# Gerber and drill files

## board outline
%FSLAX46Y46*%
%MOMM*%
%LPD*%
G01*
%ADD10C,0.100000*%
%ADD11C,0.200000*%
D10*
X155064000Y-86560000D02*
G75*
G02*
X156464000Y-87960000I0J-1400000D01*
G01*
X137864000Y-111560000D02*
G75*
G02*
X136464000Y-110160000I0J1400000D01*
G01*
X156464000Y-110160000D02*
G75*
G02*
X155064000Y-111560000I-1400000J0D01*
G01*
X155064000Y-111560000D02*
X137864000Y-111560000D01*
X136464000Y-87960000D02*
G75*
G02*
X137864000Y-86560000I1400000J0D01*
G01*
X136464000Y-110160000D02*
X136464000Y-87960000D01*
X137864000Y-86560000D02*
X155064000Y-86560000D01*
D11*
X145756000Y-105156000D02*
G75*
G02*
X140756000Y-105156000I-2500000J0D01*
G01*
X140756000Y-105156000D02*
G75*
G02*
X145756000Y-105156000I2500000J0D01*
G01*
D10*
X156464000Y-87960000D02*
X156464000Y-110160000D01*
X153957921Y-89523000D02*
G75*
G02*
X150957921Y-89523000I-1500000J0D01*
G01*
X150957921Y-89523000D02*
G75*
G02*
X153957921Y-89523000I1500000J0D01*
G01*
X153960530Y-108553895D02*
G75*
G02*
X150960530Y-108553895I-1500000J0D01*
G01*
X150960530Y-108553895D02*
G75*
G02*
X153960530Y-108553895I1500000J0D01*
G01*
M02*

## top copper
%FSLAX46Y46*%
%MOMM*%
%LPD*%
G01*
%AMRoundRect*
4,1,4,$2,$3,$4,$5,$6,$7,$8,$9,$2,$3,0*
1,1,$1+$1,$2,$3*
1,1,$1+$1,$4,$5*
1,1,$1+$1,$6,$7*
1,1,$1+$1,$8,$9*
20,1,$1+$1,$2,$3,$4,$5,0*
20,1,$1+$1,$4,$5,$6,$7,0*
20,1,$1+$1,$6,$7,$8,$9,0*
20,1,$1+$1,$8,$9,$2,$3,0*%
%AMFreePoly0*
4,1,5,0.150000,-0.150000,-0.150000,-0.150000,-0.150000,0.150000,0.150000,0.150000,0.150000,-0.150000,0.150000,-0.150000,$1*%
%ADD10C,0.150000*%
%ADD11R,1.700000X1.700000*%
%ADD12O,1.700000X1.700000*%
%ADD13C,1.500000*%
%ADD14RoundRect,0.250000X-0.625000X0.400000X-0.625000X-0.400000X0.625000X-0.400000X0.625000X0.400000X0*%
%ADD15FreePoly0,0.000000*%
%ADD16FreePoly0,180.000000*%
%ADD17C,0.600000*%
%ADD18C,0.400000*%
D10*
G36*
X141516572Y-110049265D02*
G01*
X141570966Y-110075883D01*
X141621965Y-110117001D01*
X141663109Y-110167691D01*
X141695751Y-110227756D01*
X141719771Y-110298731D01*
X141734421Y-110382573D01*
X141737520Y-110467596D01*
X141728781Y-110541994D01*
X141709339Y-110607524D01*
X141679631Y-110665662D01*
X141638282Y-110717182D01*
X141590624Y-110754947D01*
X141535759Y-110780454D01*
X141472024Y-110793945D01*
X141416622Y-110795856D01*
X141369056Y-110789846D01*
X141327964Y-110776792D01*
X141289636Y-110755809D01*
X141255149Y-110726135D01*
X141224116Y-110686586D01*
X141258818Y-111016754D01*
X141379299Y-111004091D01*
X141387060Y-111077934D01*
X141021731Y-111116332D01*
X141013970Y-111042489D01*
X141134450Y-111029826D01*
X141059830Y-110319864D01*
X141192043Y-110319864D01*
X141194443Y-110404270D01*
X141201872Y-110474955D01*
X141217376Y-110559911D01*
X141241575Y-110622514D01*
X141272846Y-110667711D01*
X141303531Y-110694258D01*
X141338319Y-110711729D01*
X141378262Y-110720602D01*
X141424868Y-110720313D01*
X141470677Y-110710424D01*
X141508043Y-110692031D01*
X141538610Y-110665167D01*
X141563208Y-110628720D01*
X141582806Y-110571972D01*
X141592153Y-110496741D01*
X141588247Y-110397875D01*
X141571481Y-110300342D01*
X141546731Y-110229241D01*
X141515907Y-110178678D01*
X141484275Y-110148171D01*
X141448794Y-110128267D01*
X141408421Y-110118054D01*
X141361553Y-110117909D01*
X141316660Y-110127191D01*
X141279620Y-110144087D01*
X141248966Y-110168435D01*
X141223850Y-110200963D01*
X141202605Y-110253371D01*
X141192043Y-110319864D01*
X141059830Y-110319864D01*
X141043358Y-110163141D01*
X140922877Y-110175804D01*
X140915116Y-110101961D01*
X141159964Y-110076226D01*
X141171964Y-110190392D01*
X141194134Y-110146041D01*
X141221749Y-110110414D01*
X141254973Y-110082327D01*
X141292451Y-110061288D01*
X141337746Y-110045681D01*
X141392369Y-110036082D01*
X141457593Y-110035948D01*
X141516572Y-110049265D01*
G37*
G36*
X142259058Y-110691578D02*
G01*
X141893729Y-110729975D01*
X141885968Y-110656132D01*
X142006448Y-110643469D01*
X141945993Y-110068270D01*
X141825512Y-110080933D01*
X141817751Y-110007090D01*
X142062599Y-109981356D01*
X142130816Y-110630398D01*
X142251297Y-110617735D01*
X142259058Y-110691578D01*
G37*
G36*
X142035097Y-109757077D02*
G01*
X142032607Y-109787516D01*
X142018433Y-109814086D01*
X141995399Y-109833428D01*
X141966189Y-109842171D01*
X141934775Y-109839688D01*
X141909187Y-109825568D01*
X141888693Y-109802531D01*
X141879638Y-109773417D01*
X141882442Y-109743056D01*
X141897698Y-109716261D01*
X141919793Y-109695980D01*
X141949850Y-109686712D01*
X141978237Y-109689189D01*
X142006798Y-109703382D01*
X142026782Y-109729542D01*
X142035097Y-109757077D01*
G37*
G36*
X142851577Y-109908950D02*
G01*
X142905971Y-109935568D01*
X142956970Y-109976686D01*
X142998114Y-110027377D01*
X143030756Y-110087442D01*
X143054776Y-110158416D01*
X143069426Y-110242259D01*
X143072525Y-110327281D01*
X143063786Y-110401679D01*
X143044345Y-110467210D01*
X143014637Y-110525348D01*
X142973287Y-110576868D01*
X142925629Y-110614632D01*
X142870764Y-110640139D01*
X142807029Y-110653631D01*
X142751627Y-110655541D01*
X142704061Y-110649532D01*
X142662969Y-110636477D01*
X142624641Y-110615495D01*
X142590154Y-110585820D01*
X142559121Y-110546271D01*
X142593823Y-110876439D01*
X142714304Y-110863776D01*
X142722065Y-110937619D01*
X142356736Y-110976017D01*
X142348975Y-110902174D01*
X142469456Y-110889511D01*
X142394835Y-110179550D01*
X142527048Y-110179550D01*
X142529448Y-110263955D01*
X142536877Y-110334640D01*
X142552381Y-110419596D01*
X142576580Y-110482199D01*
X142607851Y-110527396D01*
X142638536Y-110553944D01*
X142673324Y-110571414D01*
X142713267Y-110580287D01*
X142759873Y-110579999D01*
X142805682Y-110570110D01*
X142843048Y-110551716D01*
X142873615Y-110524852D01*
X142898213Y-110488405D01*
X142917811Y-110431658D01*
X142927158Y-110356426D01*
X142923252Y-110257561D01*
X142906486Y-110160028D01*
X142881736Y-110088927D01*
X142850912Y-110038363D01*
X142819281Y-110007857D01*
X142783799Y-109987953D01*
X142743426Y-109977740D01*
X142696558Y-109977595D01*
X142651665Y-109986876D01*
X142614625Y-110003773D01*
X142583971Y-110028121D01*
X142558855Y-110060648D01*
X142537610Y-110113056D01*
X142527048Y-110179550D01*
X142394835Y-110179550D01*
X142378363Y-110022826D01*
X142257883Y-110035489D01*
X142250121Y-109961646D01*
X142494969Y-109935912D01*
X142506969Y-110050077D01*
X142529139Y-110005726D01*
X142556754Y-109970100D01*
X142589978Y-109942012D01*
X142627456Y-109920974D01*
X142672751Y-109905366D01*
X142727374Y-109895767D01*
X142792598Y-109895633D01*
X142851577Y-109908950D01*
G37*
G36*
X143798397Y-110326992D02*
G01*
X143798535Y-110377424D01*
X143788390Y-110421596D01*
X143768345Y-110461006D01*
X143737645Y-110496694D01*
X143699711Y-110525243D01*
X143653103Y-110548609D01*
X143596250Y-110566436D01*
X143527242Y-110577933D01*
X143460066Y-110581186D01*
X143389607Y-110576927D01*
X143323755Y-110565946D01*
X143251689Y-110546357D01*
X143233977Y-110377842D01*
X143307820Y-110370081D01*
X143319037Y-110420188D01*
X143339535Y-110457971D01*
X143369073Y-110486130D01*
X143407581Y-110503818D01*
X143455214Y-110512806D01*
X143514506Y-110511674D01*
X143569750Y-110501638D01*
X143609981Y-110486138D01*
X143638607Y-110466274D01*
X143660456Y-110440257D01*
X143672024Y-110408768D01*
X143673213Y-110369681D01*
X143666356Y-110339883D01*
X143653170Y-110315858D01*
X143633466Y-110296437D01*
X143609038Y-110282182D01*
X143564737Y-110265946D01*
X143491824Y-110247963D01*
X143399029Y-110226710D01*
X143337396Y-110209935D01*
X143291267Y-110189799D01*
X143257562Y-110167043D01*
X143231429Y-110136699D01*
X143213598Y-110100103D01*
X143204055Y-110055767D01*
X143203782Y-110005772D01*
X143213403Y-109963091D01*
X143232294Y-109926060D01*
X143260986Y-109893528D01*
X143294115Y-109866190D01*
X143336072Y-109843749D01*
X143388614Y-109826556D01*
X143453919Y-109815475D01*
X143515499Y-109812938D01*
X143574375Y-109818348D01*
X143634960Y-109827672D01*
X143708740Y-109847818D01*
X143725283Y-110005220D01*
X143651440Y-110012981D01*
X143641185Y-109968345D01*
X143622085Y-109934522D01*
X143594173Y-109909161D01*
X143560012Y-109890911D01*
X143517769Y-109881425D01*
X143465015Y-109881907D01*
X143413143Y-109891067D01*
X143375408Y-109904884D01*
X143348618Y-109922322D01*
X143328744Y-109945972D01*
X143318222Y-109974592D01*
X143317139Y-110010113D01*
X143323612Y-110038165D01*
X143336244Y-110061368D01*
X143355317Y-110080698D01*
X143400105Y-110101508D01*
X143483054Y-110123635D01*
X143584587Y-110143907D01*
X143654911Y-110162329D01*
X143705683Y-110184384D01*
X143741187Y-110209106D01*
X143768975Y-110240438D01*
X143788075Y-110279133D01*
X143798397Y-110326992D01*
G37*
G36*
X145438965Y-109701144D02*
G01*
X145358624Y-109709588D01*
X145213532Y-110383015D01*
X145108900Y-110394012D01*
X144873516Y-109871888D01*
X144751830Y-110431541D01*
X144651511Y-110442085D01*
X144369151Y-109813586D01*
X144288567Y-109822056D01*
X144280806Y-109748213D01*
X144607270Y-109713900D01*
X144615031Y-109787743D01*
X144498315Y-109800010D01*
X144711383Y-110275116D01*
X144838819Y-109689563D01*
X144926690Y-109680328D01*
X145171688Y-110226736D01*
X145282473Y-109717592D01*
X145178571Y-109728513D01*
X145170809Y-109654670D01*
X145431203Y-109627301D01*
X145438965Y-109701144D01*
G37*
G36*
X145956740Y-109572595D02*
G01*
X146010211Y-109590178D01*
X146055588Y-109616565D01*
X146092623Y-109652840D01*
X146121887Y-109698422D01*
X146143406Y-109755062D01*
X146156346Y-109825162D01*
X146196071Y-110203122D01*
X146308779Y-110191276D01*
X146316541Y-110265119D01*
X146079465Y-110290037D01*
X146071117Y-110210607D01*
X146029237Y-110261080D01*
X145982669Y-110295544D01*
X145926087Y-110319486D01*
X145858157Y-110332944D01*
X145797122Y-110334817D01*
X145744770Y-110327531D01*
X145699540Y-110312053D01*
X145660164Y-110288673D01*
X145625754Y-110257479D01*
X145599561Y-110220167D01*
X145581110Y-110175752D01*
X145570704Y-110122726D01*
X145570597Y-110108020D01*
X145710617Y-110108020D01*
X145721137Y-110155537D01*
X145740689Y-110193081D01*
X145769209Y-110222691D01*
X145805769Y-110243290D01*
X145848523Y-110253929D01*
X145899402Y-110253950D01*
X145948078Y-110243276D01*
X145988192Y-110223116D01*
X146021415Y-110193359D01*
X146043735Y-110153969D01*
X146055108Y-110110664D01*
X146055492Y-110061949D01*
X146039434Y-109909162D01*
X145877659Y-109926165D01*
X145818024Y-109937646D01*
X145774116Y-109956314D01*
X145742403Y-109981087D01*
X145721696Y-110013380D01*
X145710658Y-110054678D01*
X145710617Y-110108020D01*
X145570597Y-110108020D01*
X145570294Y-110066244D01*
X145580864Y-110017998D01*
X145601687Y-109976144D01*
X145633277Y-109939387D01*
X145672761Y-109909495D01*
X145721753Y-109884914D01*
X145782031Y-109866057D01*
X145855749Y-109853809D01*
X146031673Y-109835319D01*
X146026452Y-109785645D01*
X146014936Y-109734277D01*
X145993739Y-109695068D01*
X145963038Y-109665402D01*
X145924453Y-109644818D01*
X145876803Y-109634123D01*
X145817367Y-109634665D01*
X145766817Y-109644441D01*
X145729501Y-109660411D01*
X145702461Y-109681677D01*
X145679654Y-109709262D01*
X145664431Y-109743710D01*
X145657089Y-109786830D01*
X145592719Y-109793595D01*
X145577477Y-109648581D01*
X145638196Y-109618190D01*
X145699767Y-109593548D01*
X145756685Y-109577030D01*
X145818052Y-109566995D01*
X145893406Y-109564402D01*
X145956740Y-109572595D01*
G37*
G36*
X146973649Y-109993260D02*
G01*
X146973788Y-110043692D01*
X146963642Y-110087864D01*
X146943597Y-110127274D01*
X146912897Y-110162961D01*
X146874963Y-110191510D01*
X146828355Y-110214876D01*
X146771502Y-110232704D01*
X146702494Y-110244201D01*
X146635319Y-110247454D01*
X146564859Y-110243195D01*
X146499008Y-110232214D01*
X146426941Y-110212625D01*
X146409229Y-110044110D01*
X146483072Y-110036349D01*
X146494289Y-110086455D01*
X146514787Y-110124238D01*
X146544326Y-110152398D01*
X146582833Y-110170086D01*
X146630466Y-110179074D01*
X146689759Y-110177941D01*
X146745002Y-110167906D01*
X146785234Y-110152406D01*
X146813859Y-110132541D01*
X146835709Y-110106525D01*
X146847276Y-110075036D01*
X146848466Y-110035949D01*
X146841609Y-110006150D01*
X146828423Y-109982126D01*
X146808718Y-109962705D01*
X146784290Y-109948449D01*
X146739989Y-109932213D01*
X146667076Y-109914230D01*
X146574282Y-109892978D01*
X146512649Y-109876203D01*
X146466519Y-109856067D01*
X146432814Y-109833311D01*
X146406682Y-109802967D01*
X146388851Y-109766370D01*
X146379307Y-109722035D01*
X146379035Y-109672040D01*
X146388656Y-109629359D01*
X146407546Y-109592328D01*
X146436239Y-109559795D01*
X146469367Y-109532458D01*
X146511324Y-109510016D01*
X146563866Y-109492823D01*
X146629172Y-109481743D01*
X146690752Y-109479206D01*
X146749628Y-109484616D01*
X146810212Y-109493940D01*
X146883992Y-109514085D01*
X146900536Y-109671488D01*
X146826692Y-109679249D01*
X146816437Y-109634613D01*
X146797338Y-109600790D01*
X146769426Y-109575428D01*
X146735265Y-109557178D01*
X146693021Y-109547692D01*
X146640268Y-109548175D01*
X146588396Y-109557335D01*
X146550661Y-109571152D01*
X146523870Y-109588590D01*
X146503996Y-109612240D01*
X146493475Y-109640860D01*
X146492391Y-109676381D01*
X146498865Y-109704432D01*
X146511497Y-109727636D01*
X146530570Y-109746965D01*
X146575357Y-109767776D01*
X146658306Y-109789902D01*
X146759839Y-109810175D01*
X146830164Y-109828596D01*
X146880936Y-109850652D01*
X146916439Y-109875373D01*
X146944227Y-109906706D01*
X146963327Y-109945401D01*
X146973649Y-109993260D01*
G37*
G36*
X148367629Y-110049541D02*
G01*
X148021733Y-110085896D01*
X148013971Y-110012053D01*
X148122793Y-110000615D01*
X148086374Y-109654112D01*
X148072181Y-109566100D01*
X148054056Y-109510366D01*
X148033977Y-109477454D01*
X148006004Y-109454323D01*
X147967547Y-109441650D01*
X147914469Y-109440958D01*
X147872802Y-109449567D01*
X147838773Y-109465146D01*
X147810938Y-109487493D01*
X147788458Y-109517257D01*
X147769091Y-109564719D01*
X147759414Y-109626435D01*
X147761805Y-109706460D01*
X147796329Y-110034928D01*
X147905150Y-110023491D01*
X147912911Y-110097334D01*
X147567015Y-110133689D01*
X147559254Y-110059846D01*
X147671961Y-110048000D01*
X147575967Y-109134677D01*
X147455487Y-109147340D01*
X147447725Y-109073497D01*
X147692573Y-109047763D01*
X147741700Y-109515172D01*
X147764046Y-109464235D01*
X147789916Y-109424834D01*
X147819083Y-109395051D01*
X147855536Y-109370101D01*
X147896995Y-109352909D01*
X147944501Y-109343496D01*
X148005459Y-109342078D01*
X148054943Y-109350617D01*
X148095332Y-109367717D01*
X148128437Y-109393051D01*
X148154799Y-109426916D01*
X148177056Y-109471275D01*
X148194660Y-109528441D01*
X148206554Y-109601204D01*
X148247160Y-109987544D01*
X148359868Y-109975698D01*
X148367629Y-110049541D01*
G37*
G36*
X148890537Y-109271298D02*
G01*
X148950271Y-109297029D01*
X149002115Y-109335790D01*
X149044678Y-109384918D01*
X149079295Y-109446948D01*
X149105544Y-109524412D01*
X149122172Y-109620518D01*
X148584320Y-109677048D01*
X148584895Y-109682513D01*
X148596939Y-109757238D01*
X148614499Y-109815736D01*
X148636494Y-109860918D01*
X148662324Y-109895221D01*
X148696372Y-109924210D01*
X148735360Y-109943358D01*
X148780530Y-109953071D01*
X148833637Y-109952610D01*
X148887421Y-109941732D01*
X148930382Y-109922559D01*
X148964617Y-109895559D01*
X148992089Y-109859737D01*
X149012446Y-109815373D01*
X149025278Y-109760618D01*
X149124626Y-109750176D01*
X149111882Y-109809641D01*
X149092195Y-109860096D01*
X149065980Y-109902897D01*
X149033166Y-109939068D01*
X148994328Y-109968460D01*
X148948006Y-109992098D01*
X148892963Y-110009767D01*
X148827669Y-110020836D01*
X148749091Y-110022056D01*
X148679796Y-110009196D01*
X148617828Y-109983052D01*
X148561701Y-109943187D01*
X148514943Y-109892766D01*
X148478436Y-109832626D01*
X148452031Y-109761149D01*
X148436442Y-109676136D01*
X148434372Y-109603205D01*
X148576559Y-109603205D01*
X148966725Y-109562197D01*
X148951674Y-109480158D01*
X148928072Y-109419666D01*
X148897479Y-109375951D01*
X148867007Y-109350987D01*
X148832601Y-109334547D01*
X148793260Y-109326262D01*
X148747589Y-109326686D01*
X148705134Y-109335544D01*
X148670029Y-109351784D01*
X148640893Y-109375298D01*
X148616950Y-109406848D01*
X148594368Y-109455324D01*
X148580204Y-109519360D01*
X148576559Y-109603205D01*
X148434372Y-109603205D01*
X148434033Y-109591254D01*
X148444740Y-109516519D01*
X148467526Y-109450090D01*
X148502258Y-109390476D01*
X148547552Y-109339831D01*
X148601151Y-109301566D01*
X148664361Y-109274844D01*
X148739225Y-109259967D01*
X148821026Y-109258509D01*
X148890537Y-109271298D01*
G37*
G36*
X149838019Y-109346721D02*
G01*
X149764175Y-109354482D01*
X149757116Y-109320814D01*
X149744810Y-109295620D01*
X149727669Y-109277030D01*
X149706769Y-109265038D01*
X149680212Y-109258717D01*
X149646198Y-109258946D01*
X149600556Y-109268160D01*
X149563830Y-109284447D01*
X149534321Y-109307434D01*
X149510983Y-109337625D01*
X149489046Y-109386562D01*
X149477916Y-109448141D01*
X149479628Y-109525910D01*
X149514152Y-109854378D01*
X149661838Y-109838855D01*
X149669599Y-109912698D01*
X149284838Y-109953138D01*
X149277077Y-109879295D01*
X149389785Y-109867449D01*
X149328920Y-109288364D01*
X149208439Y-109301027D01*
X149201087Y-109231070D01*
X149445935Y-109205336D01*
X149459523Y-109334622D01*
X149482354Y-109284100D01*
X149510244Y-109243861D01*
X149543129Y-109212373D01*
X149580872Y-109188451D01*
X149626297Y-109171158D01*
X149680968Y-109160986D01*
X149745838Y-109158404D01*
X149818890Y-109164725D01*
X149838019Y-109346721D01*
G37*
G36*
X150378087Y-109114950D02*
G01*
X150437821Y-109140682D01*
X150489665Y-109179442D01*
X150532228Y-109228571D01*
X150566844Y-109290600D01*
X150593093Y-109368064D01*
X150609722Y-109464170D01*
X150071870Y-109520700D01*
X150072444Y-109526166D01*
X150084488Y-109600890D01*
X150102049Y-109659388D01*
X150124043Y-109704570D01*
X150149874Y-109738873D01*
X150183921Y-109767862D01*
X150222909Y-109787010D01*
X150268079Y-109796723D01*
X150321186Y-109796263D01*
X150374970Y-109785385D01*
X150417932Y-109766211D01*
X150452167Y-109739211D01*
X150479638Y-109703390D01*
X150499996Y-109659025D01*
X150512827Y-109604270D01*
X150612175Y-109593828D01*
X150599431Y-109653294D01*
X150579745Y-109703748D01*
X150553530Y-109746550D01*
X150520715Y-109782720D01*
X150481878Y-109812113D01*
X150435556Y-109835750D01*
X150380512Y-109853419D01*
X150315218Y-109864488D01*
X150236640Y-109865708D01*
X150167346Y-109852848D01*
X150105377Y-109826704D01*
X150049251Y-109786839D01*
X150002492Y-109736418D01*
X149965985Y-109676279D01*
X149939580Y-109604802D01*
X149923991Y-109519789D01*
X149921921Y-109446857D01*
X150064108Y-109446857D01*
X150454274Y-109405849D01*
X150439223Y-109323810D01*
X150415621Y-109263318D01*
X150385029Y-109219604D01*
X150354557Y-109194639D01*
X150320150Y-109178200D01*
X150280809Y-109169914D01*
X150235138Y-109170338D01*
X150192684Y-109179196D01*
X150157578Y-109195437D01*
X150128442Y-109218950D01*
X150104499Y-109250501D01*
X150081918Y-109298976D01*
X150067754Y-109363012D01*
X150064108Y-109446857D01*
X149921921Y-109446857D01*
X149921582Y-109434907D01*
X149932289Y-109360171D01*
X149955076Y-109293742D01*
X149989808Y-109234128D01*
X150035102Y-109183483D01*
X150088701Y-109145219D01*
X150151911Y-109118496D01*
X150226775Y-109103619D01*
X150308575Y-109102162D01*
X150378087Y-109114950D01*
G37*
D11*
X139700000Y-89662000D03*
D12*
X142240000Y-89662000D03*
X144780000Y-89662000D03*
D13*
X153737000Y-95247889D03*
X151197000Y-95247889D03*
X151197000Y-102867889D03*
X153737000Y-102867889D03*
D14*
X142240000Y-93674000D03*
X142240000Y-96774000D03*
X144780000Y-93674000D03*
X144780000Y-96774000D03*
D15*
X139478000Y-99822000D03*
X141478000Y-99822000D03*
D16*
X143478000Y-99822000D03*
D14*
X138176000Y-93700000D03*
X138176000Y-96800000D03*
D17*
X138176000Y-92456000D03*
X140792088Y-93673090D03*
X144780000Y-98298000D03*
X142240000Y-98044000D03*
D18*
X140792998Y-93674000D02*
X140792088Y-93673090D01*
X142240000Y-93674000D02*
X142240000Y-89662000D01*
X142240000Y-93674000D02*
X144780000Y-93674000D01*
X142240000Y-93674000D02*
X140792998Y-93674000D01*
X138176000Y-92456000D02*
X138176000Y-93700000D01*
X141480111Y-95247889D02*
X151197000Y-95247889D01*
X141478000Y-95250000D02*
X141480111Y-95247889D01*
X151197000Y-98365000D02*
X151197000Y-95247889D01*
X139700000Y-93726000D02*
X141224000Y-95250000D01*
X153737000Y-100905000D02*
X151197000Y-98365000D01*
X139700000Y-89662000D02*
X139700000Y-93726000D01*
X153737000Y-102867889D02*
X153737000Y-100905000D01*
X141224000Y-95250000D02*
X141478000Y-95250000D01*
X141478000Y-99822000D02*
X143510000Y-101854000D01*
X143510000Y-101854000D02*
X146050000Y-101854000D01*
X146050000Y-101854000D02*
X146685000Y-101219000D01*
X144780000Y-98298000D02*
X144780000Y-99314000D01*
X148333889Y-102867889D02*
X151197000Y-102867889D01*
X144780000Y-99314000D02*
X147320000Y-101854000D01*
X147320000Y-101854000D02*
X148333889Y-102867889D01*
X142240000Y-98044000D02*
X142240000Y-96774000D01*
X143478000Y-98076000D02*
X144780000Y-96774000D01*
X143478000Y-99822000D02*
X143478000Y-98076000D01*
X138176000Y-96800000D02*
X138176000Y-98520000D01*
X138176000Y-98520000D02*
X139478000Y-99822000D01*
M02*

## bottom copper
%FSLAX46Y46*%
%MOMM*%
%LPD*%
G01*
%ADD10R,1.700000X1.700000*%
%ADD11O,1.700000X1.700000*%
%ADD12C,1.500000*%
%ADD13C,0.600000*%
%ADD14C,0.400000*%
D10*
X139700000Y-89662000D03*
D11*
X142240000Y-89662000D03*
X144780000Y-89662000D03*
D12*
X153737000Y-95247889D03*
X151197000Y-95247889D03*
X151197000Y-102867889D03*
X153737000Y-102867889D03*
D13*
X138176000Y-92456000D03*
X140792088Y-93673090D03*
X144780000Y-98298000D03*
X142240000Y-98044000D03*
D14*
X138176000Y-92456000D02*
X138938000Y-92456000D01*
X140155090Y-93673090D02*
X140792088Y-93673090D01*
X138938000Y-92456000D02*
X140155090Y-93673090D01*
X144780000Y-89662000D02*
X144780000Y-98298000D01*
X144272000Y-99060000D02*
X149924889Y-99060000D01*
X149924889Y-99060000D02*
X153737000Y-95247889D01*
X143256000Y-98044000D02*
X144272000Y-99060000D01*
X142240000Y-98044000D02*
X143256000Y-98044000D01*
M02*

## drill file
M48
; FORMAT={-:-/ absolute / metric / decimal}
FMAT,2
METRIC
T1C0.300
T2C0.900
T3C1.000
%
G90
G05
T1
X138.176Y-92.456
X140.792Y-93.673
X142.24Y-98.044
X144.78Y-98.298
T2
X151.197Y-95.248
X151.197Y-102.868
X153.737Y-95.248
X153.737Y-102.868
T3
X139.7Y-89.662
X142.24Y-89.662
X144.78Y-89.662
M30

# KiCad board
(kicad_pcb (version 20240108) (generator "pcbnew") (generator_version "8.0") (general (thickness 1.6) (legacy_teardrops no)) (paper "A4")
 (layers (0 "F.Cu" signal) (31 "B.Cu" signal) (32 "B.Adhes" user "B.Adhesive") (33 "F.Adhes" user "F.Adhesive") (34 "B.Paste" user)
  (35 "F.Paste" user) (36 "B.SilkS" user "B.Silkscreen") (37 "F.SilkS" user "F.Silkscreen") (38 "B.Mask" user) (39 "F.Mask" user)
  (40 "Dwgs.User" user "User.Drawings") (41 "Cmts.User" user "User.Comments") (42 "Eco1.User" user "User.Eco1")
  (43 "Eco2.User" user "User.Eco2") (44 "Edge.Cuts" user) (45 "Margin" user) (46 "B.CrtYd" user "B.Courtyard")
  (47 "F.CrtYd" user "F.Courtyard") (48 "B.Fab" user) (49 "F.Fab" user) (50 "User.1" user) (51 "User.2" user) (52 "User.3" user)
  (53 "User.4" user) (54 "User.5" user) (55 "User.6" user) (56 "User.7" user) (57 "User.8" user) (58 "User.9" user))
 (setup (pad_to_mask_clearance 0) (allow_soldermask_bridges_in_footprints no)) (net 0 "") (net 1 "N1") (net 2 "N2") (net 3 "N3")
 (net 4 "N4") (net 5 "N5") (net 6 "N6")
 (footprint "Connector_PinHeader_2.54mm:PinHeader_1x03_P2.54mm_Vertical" (layer "F.Cu") (at 139.7 89.662 90)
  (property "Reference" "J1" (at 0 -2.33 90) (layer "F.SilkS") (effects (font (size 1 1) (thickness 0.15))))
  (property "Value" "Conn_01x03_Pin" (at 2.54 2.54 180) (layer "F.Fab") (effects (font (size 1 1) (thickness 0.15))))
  (pad "1" thru_hole rect (at 0 0 90) (size 1.7 1.7) (drill 1) (layers "*.Cu" "*.Mask") (remove_unused_layers no) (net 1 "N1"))
  (pad "2" thru_hole oval (at 0 2.54 90) (size 1.7 1.7) (drill 1) (layers "*.Cu" "*.Mask") (remove_unused_layers no) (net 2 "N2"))
  (pad "3" thru_hole oval (at 0 5.08 90) (size 1.7 1.7) (drill 1) (layers "*.Cu" "*.Mask") (remove_unused_layers no) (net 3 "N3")))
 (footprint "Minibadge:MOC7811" (layer "F.Cu") (at 152.467 99.565889)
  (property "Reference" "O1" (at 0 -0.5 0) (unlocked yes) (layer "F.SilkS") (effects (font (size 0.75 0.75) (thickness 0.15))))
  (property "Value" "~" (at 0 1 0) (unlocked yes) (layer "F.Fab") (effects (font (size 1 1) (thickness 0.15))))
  (fp_circle (center -0.009079 -10.042889) (end 1.490921 -10.042889) (stroke (width 0.1) (type default)) (fill none) (layer "Edge.Cuts"))
  (fp_circle (center -0.00647 8.988006) (end 1.49353 8.988006) (stroke (width 0.1) (type default)) (fill none) (layer "Edge.Cuts"))
  (pad "1" thru_hole circle (at 1.27 -4.318) (size 1.5 1.5) (drill 0.9) (layers "*.Cu" "*.Mask") (remove_unused_layers no) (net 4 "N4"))
  (pad "2" thru_hole circle (at -1.27 -4.318) (size 1.5 1.5) (drill 0.9) (layers "*.Cu" "*.Mask") (remove_unused_layers no) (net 1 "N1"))
  (pad "3" thru_hole circle (at -1.27 3.302) (size 1.5 1.5) (drill 0.9) (layers "*.Cu" "*.Mask") (remove_unused_layers no) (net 3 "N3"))
  (pad "4" thru_hole circle (at 1.27 3.302) (size 1.5 1.5) (drill 0.9) (layers "*.Cu" "*.Mask") (remove_unused_layers no) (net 1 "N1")))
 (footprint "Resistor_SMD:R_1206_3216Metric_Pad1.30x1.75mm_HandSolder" (layer "F.Cu") (at 142.24 95.224 -90)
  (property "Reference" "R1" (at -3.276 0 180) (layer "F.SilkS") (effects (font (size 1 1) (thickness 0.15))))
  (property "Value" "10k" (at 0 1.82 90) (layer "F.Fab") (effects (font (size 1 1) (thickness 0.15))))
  (pad "1" smd roundrect (at -1.55 0 270) (size 1.3 1.75) (layers "F.Cu" "F.Paste" "F.Mask") (roundrect_rratio 0.192308) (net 2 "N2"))
  (pad "2" smd roundrect (at 1.55 0 270) (size 1.3 1.75) (layers "F.Cu" "F.Paste" "F.Mask") (roundrect_rratio 0.192308) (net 4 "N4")))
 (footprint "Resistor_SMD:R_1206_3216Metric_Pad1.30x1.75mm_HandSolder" (layer "F.Cu") (at 144.78 95.224 -90)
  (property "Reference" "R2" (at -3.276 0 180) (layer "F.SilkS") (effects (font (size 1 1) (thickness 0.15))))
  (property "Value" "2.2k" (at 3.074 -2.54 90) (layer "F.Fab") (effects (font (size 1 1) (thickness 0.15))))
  (pad "1" smd roundrect (at -1.55 0 270) (size 1.3 1.75) (layers "F.Cu" "F.Paste" "F.Mask") (roundrect_rratio 0.192308) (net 2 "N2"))
  (pad "2" smd roundrect (at 1.55 0 270) (size 1.3 1.75) (layers "F.Cu" "F.Paste" "F.Mask") (roundrect_rratio 0.192308) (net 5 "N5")))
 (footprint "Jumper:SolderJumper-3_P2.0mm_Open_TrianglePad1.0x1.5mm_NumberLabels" (layer "F.Cu") (at 141.478 99.822)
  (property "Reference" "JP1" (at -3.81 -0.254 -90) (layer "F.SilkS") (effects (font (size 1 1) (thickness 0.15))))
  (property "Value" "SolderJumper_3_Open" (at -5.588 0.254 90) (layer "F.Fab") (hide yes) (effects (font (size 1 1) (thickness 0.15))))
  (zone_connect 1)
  (pad "" smd rect (at -1.2 0) (size 1.5 1.5) (layers "F.Mask"))
  (pad "" smd rect (at 1.2 0) (size 1.5 1.5) (layers "F.Mask"))
  (pad "1" smd custom (at -2 0) (size 0.3 0.3) (layers "F.Cu" "F.Mask") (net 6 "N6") (zone_connect 2) (thermal_bridge_angle 45)
   (options (clearance outline) (anchor rect)) (primitives))
  (pad "2" smd custom (at 0 0) (size 0.3 0.3) (layers "F.Cu") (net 3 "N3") (zone_connect 2) (thermal_bridge_angle 45)
   (options (clearance outline) (anchor rect)) (primitives))
  (pad "3" smd custom (at 2 0 180) (size 0.3 0.3) (layers "F.Cu" "F.Mask") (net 5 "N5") (zone_connect 2) (thermal_bridge_angle 45)
   (options (clearance outline) (anchor rect)) (primitives)))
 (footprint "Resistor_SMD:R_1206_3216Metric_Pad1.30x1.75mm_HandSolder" (layer "F.Cu") (at 138.176 95.25 -90)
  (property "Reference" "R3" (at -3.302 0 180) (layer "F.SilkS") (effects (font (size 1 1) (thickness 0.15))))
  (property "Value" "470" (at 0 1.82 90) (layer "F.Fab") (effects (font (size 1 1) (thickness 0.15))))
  (pad "1" smd roundrect (at -1.55 0 270) (size 1.3 1.75) (layers "F.Cu" "F.Paste" "F.Mask") (roundrect_rratio 0.192308) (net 2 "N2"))
  (pad "2" smd roundrect (at 1.55 0 270) (size 1.3 1.75) (layers "F.Cu" "F.Paste" "F.Mask") (roundrect_rratio 0.192308) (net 6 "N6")))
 (gr_arc (start 155.064 86.56) (mid 156.053949 86.970051) (end 156.464 87.96) (stroke (width 0.1) (type default)) (layer "Edge.Cuts"))
 (gr_arc (start 137.864 111.56) (mid 136.874051 111.149949) (end 136.464 110.16) (stroke (width 0.1) (type default)) (layer "Edge.Cuts"))
 (gr_arc (start 156.464 110.16) (mid 156.053949 111.149949) (end 155.064 111.56) (stroke (width 0.1) (type default)) (layer "Edge.Cuts"))
 (gr_line (start 155.064 111.56) (end 137.864 111.56) (stroke (width 0.1) (type default)) (layer "Edge.Cuts"))
 (gr_arc (start 136.464 87.96) (mid 136.874051 86.970051) (end 137.864 86.56) (stroke (width 0.1) (type default)) (layer "Edge.Cuts"))
 (gr_line (start 136.464 110.16) (end 136.464 87.96) (stroke (width 0.1) (type default)) (layer "Edge.Cuts"))
 (gr_line (start 137.864 86.56) (end 155.064 86.56) (stroke (width 0.1) (type default)) (layer "Edge.Cuts"))
 (gr_circle (center 143.256 105.156) (end 145.756 105.156) (stroke (width 0.2) (type default)) (fill none) (layer "Edge.Cuts"))
 (gr_line (start 156.464 87.96) (end 156.464 110.16) (stroke (width 0.1) (type default)) (layer "Edge.Cuts"))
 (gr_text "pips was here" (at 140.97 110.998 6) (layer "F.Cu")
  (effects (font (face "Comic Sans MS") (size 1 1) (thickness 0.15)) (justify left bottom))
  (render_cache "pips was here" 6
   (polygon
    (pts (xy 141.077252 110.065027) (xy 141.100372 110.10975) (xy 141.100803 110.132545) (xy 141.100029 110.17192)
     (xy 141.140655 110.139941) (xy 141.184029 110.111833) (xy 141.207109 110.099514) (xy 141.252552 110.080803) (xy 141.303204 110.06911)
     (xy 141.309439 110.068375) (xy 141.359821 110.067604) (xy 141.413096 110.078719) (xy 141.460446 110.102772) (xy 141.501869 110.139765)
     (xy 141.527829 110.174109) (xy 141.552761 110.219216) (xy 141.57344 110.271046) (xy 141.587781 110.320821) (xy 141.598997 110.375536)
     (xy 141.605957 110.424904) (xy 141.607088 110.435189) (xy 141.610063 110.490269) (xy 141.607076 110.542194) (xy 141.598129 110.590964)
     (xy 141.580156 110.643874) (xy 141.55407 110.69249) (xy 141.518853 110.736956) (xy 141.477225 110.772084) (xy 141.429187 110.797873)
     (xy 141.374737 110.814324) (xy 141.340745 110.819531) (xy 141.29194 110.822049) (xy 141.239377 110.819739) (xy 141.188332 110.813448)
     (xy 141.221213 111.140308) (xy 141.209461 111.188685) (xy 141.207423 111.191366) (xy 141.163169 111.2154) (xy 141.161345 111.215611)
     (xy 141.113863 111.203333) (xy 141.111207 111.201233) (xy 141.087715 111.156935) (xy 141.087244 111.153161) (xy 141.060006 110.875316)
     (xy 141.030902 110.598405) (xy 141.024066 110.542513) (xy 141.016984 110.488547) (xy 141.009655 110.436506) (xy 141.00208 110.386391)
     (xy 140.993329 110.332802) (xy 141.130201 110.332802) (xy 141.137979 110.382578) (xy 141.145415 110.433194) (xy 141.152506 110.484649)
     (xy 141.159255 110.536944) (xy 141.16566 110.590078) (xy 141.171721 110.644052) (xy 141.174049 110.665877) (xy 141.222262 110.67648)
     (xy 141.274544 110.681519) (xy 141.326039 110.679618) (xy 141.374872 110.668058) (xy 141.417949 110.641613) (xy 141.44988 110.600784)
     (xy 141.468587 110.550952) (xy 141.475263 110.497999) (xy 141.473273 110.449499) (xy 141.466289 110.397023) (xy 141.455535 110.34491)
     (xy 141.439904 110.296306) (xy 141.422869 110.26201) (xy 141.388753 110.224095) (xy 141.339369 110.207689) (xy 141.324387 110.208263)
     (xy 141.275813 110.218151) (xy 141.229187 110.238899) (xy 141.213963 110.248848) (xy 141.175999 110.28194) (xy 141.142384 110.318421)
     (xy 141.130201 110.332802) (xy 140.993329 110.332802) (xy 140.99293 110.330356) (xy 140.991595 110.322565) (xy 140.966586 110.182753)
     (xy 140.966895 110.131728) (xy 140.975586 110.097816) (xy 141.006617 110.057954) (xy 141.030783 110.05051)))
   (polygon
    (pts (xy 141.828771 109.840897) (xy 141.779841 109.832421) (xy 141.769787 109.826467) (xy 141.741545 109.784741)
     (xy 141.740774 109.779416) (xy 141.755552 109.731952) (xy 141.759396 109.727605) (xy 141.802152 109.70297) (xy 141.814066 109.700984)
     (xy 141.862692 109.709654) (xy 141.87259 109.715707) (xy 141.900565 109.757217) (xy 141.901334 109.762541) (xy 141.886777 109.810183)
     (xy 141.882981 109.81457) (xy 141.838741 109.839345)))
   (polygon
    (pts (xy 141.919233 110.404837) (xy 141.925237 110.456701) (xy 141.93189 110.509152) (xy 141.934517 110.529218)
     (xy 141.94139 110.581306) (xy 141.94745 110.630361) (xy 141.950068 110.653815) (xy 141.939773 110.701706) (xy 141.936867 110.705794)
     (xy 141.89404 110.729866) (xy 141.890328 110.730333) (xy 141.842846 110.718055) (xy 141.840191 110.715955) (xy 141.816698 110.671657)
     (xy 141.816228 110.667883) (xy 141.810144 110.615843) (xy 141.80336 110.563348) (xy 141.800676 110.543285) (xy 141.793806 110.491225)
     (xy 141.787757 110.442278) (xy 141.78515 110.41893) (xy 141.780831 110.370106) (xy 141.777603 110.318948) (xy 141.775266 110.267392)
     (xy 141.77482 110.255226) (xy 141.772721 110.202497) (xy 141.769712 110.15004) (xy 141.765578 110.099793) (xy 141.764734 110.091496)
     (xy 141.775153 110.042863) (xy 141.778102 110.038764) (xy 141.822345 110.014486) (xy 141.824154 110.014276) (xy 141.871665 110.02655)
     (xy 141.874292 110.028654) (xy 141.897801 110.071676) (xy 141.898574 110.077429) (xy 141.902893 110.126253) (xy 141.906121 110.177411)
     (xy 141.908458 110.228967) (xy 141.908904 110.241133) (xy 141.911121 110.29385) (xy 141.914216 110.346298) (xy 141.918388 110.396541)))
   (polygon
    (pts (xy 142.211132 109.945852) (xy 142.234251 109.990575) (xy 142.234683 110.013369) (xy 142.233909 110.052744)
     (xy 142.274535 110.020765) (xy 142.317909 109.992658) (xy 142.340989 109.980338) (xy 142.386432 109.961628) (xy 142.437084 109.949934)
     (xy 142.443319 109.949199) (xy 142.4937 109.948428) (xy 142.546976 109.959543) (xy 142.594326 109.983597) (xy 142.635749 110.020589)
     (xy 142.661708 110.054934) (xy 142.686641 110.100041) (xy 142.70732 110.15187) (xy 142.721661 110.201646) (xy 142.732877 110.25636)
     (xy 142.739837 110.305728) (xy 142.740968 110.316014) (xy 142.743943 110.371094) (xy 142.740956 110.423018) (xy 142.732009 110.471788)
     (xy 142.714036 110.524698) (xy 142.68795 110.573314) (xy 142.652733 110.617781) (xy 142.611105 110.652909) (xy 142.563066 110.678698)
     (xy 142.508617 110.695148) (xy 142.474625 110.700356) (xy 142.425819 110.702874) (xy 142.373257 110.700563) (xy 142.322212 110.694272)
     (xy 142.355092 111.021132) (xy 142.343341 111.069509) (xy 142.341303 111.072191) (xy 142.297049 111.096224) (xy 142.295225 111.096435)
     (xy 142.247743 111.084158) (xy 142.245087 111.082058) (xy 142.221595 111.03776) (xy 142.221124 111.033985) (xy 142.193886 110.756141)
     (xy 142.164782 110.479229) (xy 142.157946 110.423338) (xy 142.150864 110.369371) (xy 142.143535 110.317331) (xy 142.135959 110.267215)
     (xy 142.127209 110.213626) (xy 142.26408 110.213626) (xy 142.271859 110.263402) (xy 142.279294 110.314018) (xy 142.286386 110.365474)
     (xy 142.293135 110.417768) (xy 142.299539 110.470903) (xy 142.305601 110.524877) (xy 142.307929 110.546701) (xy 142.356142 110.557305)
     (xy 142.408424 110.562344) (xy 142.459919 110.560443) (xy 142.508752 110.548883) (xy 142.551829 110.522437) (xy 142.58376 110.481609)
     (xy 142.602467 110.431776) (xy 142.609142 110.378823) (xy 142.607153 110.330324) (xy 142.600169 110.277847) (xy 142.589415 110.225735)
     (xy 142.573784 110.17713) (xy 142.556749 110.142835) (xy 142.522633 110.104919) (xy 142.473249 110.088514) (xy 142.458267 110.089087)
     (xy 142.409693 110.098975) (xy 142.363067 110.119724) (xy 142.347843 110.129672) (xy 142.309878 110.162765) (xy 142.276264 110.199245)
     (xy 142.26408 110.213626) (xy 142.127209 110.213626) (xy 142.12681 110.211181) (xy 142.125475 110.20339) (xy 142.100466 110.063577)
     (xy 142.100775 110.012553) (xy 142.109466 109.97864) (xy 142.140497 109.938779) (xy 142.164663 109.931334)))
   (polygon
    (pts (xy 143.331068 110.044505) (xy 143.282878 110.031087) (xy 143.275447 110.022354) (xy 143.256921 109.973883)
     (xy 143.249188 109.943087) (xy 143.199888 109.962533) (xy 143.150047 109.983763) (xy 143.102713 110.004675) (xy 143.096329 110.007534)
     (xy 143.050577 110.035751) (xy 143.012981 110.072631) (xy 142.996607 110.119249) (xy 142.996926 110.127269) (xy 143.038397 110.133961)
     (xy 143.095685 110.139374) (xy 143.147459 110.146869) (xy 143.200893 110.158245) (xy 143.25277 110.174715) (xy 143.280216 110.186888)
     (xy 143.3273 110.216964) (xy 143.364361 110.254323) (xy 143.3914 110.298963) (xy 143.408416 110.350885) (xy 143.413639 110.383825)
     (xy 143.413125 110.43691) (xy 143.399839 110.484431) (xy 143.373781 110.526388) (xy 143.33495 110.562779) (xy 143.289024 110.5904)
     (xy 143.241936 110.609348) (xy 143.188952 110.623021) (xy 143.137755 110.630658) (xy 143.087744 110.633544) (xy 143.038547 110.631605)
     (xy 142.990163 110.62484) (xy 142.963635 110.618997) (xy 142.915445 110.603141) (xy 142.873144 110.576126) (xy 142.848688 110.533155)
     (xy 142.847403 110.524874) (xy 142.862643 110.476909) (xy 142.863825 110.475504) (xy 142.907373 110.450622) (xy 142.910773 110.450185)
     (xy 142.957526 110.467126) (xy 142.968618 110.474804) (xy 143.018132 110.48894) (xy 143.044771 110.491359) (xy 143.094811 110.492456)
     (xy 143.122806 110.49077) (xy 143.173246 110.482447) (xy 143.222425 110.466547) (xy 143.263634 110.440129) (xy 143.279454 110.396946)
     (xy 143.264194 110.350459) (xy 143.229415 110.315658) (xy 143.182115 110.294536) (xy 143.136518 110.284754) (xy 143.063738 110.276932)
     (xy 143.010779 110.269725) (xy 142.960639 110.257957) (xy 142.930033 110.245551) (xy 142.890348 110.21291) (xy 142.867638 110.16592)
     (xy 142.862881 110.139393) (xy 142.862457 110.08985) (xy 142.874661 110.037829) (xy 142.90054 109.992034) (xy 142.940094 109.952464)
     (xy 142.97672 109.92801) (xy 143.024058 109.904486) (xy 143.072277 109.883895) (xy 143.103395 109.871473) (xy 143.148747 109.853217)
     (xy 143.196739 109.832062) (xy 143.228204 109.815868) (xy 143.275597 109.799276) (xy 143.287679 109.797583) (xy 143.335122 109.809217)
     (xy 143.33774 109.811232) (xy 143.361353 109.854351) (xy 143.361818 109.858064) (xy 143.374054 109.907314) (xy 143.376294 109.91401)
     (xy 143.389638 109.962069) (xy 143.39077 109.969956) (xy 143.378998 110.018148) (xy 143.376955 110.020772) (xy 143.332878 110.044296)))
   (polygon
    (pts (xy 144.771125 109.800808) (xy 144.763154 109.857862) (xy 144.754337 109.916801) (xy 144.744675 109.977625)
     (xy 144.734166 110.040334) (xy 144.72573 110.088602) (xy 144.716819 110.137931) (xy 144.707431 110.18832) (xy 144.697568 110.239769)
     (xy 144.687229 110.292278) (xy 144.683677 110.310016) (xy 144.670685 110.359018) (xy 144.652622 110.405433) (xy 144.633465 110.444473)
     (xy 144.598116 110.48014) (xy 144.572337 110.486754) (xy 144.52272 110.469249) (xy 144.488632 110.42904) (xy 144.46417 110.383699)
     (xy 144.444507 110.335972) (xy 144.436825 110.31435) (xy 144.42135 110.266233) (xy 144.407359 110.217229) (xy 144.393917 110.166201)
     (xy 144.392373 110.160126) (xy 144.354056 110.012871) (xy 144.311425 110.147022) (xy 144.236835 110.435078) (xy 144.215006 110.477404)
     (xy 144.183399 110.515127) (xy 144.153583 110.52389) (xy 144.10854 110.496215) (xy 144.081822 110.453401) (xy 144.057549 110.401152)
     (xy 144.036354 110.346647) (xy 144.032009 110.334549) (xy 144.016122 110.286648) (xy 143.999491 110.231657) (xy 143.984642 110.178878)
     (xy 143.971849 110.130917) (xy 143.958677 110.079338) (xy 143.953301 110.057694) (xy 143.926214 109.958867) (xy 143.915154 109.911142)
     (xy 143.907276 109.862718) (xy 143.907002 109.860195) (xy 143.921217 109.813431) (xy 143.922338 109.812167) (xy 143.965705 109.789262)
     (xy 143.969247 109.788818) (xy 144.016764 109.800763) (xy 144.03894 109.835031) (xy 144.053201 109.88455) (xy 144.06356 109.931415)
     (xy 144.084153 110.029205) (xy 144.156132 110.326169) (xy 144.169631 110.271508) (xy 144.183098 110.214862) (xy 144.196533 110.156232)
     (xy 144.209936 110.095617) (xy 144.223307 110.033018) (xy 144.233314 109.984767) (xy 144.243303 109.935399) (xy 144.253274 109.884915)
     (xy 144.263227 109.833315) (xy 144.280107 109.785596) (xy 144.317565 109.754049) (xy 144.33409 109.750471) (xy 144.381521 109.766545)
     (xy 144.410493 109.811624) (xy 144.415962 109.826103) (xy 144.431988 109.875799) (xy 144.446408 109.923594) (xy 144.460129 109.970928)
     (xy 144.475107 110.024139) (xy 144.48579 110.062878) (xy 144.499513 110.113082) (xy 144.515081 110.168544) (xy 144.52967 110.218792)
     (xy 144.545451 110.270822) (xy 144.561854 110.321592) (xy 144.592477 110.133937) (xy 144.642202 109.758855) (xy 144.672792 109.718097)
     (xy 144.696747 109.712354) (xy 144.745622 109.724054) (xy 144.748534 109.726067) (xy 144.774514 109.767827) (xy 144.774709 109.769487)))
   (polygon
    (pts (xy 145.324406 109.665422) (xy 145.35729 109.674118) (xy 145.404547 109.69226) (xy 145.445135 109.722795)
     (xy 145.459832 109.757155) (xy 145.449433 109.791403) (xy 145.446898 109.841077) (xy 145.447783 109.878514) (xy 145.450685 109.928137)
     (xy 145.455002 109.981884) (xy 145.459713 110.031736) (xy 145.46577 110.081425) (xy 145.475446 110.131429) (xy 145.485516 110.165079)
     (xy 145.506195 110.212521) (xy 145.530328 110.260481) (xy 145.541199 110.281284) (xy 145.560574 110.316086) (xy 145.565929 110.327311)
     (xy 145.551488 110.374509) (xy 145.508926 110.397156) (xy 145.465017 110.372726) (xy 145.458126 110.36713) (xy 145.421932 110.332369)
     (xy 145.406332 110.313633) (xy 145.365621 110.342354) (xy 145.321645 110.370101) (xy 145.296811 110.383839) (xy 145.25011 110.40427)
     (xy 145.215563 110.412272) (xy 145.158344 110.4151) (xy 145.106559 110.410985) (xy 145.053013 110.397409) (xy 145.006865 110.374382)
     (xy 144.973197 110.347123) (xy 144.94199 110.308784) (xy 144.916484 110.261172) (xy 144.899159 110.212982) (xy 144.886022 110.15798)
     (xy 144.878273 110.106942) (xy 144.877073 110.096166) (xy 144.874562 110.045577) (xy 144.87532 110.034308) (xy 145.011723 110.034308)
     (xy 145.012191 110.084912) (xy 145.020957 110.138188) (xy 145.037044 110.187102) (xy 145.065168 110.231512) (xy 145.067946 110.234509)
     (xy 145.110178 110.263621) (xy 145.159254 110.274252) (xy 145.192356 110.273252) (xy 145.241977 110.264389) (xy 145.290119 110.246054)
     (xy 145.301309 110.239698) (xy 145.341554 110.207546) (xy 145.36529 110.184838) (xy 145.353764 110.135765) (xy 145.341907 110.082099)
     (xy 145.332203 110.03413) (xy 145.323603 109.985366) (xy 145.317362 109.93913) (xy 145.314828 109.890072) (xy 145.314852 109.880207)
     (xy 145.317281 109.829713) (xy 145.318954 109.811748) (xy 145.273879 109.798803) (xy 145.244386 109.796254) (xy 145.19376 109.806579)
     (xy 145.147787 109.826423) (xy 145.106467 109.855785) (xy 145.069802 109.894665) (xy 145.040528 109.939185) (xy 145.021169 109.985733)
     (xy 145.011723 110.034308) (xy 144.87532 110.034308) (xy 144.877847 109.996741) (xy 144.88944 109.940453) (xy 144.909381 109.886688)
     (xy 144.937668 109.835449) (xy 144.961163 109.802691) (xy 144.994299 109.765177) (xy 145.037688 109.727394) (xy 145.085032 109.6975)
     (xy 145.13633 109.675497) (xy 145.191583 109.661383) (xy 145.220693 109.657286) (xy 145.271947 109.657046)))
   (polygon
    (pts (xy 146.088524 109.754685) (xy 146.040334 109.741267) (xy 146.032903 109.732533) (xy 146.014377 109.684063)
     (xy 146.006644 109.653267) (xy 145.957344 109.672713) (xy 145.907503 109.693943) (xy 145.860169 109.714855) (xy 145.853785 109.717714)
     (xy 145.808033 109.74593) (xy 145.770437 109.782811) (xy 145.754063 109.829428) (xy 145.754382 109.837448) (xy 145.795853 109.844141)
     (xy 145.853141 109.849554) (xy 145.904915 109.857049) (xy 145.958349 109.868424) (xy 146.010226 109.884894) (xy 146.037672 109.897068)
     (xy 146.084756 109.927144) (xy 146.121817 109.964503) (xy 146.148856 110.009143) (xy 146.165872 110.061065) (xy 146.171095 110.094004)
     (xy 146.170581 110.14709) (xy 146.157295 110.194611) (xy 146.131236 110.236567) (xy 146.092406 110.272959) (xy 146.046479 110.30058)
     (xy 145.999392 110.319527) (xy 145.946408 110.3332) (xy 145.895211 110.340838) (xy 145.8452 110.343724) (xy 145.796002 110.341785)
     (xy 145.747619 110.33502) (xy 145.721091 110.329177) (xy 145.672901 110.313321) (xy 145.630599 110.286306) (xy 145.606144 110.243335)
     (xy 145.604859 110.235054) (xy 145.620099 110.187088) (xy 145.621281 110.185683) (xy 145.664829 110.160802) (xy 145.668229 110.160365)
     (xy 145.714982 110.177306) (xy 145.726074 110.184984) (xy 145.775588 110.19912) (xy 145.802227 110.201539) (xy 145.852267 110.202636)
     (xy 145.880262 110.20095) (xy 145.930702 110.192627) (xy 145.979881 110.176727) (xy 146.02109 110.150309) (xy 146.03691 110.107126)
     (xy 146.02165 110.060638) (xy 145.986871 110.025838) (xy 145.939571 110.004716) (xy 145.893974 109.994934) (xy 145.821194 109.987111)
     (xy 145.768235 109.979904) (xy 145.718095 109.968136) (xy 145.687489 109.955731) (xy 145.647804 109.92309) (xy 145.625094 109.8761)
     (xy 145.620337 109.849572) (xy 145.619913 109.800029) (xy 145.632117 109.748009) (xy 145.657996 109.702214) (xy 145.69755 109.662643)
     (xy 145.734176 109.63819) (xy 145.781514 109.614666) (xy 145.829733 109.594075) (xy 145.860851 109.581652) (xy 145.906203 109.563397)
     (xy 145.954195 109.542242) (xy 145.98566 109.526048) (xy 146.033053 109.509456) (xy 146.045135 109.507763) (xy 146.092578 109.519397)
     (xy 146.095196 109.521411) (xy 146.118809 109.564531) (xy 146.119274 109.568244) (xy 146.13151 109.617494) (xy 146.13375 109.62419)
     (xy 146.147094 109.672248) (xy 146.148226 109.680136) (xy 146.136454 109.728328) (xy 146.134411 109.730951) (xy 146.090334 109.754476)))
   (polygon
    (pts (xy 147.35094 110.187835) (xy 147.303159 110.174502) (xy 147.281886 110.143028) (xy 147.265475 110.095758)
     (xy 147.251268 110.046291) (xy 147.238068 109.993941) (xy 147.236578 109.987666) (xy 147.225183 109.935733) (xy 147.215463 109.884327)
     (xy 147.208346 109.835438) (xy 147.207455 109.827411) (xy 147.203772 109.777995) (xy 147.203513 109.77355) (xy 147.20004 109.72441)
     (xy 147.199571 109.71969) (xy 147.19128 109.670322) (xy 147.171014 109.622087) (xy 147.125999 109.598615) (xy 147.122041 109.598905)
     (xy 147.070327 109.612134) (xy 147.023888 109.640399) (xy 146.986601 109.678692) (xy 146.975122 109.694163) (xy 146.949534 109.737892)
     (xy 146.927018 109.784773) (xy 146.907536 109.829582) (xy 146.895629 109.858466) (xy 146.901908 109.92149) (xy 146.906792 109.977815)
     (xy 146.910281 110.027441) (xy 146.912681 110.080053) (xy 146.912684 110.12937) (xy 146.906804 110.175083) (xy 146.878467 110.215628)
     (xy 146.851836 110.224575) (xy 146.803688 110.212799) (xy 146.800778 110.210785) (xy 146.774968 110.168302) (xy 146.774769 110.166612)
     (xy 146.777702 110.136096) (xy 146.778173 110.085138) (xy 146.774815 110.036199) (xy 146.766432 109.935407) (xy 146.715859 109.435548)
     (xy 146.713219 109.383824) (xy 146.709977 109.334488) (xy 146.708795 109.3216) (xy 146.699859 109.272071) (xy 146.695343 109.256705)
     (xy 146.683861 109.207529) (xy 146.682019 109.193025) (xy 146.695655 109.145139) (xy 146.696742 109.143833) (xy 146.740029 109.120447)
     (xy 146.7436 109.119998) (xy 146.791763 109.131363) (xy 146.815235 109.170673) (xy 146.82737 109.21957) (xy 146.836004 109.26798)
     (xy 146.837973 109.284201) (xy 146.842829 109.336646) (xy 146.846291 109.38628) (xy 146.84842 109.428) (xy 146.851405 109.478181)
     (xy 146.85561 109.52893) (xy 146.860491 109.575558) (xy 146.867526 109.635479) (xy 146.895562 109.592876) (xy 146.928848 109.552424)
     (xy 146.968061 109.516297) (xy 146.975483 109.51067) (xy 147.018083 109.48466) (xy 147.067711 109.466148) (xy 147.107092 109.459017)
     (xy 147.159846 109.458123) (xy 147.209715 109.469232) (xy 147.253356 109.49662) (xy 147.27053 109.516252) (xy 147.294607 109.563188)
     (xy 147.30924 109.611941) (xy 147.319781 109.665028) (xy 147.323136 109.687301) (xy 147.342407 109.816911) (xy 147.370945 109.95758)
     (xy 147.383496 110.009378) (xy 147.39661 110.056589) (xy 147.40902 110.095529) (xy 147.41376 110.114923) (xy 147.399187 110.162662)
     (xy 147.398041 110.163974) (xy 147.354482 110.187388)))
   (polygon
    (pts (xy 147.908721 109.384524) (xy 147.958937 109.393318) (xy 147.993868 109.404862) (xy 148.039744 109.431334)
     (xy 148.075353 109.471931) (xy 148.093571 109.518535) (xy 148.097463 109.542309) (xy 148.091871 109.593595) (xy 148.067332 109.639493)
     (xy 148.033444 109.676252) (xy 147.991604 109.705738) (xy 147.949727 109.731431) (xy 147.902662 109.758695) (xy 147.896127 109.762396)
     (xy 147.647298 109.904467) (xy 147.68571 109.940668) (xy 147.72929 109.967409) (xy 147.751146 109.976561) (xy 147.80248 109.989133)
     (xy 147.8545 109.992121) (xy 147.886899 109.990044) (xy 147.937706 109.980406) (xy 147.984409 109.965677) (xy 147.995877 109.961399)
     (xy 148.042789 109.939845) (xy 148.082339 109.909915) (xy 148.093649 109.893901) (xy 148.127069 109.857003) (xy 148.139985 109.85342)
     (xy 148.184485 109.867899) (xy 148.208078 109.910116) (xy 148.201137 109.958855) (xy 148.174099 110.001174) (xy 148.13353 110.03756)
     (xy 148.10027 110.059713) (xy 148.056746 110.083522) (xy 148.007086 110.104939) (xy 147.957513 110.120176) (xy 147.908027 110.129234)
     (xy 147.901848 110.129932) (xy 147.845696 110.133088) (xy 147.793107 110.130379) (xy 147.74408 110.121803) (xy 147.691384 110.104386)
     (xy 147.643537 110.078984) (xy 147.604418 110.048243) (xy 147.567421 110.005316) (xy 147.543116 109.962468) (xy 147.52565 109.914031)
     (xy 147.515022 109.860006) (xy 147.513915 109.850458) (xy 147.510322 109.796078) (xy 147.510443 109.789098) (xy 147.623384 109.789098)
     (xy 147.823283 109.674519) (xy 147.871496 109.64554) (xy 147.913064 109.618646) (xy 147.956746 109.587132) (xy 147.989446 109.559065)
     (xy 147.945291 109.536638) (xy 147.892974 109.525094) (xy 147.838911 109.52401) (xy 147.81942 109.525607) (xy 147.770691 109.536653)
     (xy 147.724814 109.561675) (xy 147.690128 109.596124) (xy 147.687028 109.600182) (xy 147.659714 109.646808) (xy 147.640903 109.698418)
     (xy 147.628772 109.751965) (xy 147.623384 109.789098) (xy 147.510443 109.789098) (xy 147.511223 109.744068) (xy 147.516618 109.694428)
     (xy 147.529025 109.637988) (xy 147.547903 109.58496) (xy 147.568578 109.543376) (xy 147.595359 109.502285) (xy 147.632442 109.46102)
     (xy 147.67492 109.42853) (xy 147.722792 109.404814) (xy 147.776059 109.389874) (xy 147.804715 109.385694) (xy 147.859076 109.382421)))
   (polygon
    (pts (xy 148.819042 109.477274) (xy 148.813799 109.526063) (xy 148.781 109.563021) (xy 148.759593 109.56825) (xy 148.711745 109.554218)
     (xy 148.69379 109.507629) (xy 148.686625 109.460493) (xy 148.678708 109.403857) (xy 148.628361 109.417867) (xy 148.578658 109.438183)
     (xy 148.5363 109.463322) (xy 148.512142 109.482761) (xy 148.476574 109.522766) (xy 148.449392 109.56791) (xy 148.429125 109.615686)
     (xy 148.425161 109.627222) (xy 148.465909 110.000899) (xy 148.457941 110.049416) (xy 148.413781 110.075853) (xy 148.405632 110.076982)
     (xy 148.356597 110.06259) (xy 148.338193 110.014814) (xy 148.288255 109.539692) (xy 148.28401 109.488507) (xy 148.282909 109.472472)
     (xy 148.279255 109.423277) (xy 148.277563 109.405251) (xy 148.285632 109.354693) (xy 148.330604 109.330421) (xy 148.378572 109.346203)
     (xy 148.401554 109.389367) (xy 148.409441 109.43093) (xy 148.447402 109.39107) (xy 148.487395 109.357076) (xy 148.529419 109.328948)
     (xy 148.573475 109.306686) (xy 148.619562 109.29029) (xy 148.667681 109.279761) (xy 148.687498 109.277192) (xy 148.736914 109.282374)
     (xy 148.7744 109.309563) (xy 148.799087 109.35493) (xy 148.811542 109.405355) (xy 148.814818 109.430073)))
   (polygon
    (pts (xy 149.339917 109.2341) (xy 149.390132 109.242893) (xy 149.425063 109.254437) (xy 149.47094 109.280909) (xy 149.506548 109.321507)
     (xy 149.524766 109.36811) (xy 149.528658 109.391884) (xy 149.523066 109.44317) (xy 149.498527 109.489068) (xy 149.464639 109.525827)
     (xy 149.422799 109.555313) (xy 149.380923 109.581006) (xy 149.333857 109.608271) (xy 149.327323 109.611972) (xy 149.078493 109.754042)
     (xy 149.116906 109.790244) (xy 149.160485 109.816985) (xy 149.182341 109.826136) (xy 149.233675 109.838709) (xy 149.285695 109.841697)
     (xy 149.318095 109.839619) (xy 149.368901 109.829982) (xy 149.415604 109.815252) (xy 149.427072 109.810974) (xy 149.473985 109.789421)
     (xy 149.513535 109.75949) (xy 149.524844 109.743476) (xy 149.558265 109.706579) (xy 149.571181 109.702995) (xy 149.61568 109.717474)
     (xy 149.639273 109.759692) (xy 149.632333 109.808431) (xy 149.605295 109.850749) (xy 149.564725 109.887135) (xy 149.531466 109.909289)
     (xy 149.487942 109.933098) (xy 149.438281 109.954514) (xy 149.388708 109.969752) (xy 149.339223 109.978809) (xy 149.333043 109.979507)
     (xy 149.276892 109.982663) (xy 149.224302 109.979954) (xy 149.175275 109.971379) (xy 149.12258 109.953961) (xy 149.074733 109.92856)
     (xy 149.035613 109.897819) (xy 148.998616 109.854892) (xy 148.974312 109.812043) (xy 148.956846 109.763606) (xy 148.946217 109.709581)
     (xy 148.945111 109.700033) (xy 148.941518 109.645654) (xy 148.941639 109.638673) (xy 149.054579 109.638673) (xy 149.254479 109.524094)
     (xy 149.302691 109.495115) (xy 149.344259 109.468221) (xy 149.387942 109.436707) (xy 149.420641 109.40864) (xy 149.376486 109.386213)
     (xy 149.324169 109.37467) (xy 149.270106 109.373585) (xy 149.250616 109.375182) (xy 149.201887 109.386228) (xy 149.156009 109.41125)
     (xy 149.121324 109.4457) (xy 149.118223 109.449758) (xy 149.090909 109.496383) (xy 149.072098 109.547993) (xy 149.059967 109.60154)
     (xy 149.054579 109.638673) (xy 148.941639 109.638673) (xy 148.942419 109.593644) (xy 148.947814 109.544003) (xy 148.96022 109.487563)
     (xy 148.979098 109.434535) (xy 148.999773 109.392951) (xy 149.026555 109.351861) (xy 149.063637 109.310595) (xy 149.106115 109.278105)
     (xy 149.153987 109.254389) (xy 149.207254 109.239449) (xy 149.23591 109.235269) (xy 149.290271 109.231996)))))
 (segment (start 140.792998 93.674) (end 140.792088 93.67309) (width 0.4) (layer "F.Cu") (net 2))
 (segment (start 142.24 93.674) (end 142.24 89.662) (width 0.4) (layer "F.Cu") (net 2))
 (segment (start 142.24 93.674) (end 144.78 93.674) (width 0.4) (layer "F.Cu") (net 2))
 (segment (start 142.24 93.674) (end 140.792998 93.674) (width 0.4) (layer "F.Cu") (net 2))
 (segment (start 138.176 92.456) (end 138.176 93.7) (width 0.4) (layer "F.Cu") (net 2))
 (via (at 138.176 92.456) (size 0.6) (drill 0.3) (layers "F.Cu" "B.Cu") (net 2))
 (via (at 140.792088 93.67309) (size 0.6) (drill 0.3) (layers "F.Cu" "B.Cu") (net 2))
 (segment (start 138.176 92.456) (end 138.938 92.456) (width 0.4) (layer "B.Cu") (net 2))
 (segment (start 140.15509 93.67309) (end 140.792088 93.67309) (width 0.4) (layer "B.Cu") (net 2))
 (segment (start 138.938 92.456) (end 140.15509 93.67309) (width 0.4) (layer "B.Cu") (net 2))
 (segment (start 141.480111 95.247889) (end 151.197 95.247889) (width 0.4) (layer "F.Cu") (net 1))
 (segment (start 141.478 95.25) (end 141.480111 95.247889) (width 0.4) (layer "F.Cu") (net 1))
 (segment (start 151.197 98.365) (end 151.197 95.247889) (width 0.4) (layer "F.Cu") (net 1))
 (segment (start 139.7 93.726) (end 141.224 95.25) (width 0.4) (layer "F.Cu") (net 1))
 (segment (start 153.737 100.905) (end 151.197 98.365) (width 0.4) (layer "F.Cu") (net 1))
 (segment (start 139.7 89.662) (end 139.7 93.726) (width 0.4) (layer "F.Cu") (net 1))
 (segment (start 153.737 102.867889) (end 153.737 100.905) (width 0.4) (layer "F.Cu") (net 1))
 (segment (start 141.224 95.25) (end 141.478 95.25) (width 0.4) (layer "F.Cu") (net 1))
 (segment (start 141.478 99.822) (end 143.51 101.854) (width 0.4) (layer "F.Cu") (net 3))
 (segment (start 143.51 101.854) (end 146.05 101.854) (width 0.4) (layer "F.Cu") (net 3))
 (segment (start 146.05 101.854) (end 146.685 101.219) (width 0.4) (layer "F.Cu") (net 3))
 (segment (start 144.78 98.298) (end 144.78 99.314) (width 0.4) (layer "F.Cu") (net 3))
 (segment (start 148.333889 102.867889) (end 151.197 102.867889) (width 0.4) (layer "F.Cu") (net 3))
 (segment (start 144.78 99.314) (end 147.32 101.854) (width 0.4) (layer "F.Cu") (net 3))
 (segment (start 147.32 101.854) (end 148.333889 102.867889) (width 0.4) (layer "F.Cu") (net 3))
 (via (at 144.78 98.298) (size 0.6) (drill 0.3) (layers "F.Cu" "B.Cu") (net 3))
 (segment (start 144.78 89.662) (end 144.78 98.298) (width 0.4) (layer "B.Cu") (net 3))
 (segment (start 142.24 98.044) (end 142.24 96.774) (width 0.4) (layer "F.Cu") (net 4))
 (via (at 142.24 98.044) (size 0.6) (drill 0.3) (layers "F.Cu" "B.Cu") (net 4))
 (segment (start 144.272 99.06) (end 149.924889 99.06) (width 0.4) (layer "B.Cu") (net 4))
 (segment (start 149.924889 99.06) (end 153.737 95.247889) (width 0.4) (layer "B.Cu") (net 4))
 (segment (start 143.256 98.044) (end 144.272 99.06) (width 0.4) (layer "B.Cu") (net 4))
 (segment (start 142.24 98.044) (end 143.256 98.044) (width 0.4) (layer "B.Cu") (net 4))
 (segment (start 143.478 98.076) (end 144.78 96.774) (width 0.4) (layer "F.Cu") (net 5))
 (segment (start 143.478 99.822) (end 143.478 98.076) (width 0.4) (layer "F.Cu") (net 5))
 (segment (start 138.176 96.8) (end 138.176 98.52) (width 0.4) (layer "F.Cu") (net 6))
 (segment (start 138.176 98.52) (end 139.478 99.822) (width 0.4) (layer "F.Cu") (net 6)))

